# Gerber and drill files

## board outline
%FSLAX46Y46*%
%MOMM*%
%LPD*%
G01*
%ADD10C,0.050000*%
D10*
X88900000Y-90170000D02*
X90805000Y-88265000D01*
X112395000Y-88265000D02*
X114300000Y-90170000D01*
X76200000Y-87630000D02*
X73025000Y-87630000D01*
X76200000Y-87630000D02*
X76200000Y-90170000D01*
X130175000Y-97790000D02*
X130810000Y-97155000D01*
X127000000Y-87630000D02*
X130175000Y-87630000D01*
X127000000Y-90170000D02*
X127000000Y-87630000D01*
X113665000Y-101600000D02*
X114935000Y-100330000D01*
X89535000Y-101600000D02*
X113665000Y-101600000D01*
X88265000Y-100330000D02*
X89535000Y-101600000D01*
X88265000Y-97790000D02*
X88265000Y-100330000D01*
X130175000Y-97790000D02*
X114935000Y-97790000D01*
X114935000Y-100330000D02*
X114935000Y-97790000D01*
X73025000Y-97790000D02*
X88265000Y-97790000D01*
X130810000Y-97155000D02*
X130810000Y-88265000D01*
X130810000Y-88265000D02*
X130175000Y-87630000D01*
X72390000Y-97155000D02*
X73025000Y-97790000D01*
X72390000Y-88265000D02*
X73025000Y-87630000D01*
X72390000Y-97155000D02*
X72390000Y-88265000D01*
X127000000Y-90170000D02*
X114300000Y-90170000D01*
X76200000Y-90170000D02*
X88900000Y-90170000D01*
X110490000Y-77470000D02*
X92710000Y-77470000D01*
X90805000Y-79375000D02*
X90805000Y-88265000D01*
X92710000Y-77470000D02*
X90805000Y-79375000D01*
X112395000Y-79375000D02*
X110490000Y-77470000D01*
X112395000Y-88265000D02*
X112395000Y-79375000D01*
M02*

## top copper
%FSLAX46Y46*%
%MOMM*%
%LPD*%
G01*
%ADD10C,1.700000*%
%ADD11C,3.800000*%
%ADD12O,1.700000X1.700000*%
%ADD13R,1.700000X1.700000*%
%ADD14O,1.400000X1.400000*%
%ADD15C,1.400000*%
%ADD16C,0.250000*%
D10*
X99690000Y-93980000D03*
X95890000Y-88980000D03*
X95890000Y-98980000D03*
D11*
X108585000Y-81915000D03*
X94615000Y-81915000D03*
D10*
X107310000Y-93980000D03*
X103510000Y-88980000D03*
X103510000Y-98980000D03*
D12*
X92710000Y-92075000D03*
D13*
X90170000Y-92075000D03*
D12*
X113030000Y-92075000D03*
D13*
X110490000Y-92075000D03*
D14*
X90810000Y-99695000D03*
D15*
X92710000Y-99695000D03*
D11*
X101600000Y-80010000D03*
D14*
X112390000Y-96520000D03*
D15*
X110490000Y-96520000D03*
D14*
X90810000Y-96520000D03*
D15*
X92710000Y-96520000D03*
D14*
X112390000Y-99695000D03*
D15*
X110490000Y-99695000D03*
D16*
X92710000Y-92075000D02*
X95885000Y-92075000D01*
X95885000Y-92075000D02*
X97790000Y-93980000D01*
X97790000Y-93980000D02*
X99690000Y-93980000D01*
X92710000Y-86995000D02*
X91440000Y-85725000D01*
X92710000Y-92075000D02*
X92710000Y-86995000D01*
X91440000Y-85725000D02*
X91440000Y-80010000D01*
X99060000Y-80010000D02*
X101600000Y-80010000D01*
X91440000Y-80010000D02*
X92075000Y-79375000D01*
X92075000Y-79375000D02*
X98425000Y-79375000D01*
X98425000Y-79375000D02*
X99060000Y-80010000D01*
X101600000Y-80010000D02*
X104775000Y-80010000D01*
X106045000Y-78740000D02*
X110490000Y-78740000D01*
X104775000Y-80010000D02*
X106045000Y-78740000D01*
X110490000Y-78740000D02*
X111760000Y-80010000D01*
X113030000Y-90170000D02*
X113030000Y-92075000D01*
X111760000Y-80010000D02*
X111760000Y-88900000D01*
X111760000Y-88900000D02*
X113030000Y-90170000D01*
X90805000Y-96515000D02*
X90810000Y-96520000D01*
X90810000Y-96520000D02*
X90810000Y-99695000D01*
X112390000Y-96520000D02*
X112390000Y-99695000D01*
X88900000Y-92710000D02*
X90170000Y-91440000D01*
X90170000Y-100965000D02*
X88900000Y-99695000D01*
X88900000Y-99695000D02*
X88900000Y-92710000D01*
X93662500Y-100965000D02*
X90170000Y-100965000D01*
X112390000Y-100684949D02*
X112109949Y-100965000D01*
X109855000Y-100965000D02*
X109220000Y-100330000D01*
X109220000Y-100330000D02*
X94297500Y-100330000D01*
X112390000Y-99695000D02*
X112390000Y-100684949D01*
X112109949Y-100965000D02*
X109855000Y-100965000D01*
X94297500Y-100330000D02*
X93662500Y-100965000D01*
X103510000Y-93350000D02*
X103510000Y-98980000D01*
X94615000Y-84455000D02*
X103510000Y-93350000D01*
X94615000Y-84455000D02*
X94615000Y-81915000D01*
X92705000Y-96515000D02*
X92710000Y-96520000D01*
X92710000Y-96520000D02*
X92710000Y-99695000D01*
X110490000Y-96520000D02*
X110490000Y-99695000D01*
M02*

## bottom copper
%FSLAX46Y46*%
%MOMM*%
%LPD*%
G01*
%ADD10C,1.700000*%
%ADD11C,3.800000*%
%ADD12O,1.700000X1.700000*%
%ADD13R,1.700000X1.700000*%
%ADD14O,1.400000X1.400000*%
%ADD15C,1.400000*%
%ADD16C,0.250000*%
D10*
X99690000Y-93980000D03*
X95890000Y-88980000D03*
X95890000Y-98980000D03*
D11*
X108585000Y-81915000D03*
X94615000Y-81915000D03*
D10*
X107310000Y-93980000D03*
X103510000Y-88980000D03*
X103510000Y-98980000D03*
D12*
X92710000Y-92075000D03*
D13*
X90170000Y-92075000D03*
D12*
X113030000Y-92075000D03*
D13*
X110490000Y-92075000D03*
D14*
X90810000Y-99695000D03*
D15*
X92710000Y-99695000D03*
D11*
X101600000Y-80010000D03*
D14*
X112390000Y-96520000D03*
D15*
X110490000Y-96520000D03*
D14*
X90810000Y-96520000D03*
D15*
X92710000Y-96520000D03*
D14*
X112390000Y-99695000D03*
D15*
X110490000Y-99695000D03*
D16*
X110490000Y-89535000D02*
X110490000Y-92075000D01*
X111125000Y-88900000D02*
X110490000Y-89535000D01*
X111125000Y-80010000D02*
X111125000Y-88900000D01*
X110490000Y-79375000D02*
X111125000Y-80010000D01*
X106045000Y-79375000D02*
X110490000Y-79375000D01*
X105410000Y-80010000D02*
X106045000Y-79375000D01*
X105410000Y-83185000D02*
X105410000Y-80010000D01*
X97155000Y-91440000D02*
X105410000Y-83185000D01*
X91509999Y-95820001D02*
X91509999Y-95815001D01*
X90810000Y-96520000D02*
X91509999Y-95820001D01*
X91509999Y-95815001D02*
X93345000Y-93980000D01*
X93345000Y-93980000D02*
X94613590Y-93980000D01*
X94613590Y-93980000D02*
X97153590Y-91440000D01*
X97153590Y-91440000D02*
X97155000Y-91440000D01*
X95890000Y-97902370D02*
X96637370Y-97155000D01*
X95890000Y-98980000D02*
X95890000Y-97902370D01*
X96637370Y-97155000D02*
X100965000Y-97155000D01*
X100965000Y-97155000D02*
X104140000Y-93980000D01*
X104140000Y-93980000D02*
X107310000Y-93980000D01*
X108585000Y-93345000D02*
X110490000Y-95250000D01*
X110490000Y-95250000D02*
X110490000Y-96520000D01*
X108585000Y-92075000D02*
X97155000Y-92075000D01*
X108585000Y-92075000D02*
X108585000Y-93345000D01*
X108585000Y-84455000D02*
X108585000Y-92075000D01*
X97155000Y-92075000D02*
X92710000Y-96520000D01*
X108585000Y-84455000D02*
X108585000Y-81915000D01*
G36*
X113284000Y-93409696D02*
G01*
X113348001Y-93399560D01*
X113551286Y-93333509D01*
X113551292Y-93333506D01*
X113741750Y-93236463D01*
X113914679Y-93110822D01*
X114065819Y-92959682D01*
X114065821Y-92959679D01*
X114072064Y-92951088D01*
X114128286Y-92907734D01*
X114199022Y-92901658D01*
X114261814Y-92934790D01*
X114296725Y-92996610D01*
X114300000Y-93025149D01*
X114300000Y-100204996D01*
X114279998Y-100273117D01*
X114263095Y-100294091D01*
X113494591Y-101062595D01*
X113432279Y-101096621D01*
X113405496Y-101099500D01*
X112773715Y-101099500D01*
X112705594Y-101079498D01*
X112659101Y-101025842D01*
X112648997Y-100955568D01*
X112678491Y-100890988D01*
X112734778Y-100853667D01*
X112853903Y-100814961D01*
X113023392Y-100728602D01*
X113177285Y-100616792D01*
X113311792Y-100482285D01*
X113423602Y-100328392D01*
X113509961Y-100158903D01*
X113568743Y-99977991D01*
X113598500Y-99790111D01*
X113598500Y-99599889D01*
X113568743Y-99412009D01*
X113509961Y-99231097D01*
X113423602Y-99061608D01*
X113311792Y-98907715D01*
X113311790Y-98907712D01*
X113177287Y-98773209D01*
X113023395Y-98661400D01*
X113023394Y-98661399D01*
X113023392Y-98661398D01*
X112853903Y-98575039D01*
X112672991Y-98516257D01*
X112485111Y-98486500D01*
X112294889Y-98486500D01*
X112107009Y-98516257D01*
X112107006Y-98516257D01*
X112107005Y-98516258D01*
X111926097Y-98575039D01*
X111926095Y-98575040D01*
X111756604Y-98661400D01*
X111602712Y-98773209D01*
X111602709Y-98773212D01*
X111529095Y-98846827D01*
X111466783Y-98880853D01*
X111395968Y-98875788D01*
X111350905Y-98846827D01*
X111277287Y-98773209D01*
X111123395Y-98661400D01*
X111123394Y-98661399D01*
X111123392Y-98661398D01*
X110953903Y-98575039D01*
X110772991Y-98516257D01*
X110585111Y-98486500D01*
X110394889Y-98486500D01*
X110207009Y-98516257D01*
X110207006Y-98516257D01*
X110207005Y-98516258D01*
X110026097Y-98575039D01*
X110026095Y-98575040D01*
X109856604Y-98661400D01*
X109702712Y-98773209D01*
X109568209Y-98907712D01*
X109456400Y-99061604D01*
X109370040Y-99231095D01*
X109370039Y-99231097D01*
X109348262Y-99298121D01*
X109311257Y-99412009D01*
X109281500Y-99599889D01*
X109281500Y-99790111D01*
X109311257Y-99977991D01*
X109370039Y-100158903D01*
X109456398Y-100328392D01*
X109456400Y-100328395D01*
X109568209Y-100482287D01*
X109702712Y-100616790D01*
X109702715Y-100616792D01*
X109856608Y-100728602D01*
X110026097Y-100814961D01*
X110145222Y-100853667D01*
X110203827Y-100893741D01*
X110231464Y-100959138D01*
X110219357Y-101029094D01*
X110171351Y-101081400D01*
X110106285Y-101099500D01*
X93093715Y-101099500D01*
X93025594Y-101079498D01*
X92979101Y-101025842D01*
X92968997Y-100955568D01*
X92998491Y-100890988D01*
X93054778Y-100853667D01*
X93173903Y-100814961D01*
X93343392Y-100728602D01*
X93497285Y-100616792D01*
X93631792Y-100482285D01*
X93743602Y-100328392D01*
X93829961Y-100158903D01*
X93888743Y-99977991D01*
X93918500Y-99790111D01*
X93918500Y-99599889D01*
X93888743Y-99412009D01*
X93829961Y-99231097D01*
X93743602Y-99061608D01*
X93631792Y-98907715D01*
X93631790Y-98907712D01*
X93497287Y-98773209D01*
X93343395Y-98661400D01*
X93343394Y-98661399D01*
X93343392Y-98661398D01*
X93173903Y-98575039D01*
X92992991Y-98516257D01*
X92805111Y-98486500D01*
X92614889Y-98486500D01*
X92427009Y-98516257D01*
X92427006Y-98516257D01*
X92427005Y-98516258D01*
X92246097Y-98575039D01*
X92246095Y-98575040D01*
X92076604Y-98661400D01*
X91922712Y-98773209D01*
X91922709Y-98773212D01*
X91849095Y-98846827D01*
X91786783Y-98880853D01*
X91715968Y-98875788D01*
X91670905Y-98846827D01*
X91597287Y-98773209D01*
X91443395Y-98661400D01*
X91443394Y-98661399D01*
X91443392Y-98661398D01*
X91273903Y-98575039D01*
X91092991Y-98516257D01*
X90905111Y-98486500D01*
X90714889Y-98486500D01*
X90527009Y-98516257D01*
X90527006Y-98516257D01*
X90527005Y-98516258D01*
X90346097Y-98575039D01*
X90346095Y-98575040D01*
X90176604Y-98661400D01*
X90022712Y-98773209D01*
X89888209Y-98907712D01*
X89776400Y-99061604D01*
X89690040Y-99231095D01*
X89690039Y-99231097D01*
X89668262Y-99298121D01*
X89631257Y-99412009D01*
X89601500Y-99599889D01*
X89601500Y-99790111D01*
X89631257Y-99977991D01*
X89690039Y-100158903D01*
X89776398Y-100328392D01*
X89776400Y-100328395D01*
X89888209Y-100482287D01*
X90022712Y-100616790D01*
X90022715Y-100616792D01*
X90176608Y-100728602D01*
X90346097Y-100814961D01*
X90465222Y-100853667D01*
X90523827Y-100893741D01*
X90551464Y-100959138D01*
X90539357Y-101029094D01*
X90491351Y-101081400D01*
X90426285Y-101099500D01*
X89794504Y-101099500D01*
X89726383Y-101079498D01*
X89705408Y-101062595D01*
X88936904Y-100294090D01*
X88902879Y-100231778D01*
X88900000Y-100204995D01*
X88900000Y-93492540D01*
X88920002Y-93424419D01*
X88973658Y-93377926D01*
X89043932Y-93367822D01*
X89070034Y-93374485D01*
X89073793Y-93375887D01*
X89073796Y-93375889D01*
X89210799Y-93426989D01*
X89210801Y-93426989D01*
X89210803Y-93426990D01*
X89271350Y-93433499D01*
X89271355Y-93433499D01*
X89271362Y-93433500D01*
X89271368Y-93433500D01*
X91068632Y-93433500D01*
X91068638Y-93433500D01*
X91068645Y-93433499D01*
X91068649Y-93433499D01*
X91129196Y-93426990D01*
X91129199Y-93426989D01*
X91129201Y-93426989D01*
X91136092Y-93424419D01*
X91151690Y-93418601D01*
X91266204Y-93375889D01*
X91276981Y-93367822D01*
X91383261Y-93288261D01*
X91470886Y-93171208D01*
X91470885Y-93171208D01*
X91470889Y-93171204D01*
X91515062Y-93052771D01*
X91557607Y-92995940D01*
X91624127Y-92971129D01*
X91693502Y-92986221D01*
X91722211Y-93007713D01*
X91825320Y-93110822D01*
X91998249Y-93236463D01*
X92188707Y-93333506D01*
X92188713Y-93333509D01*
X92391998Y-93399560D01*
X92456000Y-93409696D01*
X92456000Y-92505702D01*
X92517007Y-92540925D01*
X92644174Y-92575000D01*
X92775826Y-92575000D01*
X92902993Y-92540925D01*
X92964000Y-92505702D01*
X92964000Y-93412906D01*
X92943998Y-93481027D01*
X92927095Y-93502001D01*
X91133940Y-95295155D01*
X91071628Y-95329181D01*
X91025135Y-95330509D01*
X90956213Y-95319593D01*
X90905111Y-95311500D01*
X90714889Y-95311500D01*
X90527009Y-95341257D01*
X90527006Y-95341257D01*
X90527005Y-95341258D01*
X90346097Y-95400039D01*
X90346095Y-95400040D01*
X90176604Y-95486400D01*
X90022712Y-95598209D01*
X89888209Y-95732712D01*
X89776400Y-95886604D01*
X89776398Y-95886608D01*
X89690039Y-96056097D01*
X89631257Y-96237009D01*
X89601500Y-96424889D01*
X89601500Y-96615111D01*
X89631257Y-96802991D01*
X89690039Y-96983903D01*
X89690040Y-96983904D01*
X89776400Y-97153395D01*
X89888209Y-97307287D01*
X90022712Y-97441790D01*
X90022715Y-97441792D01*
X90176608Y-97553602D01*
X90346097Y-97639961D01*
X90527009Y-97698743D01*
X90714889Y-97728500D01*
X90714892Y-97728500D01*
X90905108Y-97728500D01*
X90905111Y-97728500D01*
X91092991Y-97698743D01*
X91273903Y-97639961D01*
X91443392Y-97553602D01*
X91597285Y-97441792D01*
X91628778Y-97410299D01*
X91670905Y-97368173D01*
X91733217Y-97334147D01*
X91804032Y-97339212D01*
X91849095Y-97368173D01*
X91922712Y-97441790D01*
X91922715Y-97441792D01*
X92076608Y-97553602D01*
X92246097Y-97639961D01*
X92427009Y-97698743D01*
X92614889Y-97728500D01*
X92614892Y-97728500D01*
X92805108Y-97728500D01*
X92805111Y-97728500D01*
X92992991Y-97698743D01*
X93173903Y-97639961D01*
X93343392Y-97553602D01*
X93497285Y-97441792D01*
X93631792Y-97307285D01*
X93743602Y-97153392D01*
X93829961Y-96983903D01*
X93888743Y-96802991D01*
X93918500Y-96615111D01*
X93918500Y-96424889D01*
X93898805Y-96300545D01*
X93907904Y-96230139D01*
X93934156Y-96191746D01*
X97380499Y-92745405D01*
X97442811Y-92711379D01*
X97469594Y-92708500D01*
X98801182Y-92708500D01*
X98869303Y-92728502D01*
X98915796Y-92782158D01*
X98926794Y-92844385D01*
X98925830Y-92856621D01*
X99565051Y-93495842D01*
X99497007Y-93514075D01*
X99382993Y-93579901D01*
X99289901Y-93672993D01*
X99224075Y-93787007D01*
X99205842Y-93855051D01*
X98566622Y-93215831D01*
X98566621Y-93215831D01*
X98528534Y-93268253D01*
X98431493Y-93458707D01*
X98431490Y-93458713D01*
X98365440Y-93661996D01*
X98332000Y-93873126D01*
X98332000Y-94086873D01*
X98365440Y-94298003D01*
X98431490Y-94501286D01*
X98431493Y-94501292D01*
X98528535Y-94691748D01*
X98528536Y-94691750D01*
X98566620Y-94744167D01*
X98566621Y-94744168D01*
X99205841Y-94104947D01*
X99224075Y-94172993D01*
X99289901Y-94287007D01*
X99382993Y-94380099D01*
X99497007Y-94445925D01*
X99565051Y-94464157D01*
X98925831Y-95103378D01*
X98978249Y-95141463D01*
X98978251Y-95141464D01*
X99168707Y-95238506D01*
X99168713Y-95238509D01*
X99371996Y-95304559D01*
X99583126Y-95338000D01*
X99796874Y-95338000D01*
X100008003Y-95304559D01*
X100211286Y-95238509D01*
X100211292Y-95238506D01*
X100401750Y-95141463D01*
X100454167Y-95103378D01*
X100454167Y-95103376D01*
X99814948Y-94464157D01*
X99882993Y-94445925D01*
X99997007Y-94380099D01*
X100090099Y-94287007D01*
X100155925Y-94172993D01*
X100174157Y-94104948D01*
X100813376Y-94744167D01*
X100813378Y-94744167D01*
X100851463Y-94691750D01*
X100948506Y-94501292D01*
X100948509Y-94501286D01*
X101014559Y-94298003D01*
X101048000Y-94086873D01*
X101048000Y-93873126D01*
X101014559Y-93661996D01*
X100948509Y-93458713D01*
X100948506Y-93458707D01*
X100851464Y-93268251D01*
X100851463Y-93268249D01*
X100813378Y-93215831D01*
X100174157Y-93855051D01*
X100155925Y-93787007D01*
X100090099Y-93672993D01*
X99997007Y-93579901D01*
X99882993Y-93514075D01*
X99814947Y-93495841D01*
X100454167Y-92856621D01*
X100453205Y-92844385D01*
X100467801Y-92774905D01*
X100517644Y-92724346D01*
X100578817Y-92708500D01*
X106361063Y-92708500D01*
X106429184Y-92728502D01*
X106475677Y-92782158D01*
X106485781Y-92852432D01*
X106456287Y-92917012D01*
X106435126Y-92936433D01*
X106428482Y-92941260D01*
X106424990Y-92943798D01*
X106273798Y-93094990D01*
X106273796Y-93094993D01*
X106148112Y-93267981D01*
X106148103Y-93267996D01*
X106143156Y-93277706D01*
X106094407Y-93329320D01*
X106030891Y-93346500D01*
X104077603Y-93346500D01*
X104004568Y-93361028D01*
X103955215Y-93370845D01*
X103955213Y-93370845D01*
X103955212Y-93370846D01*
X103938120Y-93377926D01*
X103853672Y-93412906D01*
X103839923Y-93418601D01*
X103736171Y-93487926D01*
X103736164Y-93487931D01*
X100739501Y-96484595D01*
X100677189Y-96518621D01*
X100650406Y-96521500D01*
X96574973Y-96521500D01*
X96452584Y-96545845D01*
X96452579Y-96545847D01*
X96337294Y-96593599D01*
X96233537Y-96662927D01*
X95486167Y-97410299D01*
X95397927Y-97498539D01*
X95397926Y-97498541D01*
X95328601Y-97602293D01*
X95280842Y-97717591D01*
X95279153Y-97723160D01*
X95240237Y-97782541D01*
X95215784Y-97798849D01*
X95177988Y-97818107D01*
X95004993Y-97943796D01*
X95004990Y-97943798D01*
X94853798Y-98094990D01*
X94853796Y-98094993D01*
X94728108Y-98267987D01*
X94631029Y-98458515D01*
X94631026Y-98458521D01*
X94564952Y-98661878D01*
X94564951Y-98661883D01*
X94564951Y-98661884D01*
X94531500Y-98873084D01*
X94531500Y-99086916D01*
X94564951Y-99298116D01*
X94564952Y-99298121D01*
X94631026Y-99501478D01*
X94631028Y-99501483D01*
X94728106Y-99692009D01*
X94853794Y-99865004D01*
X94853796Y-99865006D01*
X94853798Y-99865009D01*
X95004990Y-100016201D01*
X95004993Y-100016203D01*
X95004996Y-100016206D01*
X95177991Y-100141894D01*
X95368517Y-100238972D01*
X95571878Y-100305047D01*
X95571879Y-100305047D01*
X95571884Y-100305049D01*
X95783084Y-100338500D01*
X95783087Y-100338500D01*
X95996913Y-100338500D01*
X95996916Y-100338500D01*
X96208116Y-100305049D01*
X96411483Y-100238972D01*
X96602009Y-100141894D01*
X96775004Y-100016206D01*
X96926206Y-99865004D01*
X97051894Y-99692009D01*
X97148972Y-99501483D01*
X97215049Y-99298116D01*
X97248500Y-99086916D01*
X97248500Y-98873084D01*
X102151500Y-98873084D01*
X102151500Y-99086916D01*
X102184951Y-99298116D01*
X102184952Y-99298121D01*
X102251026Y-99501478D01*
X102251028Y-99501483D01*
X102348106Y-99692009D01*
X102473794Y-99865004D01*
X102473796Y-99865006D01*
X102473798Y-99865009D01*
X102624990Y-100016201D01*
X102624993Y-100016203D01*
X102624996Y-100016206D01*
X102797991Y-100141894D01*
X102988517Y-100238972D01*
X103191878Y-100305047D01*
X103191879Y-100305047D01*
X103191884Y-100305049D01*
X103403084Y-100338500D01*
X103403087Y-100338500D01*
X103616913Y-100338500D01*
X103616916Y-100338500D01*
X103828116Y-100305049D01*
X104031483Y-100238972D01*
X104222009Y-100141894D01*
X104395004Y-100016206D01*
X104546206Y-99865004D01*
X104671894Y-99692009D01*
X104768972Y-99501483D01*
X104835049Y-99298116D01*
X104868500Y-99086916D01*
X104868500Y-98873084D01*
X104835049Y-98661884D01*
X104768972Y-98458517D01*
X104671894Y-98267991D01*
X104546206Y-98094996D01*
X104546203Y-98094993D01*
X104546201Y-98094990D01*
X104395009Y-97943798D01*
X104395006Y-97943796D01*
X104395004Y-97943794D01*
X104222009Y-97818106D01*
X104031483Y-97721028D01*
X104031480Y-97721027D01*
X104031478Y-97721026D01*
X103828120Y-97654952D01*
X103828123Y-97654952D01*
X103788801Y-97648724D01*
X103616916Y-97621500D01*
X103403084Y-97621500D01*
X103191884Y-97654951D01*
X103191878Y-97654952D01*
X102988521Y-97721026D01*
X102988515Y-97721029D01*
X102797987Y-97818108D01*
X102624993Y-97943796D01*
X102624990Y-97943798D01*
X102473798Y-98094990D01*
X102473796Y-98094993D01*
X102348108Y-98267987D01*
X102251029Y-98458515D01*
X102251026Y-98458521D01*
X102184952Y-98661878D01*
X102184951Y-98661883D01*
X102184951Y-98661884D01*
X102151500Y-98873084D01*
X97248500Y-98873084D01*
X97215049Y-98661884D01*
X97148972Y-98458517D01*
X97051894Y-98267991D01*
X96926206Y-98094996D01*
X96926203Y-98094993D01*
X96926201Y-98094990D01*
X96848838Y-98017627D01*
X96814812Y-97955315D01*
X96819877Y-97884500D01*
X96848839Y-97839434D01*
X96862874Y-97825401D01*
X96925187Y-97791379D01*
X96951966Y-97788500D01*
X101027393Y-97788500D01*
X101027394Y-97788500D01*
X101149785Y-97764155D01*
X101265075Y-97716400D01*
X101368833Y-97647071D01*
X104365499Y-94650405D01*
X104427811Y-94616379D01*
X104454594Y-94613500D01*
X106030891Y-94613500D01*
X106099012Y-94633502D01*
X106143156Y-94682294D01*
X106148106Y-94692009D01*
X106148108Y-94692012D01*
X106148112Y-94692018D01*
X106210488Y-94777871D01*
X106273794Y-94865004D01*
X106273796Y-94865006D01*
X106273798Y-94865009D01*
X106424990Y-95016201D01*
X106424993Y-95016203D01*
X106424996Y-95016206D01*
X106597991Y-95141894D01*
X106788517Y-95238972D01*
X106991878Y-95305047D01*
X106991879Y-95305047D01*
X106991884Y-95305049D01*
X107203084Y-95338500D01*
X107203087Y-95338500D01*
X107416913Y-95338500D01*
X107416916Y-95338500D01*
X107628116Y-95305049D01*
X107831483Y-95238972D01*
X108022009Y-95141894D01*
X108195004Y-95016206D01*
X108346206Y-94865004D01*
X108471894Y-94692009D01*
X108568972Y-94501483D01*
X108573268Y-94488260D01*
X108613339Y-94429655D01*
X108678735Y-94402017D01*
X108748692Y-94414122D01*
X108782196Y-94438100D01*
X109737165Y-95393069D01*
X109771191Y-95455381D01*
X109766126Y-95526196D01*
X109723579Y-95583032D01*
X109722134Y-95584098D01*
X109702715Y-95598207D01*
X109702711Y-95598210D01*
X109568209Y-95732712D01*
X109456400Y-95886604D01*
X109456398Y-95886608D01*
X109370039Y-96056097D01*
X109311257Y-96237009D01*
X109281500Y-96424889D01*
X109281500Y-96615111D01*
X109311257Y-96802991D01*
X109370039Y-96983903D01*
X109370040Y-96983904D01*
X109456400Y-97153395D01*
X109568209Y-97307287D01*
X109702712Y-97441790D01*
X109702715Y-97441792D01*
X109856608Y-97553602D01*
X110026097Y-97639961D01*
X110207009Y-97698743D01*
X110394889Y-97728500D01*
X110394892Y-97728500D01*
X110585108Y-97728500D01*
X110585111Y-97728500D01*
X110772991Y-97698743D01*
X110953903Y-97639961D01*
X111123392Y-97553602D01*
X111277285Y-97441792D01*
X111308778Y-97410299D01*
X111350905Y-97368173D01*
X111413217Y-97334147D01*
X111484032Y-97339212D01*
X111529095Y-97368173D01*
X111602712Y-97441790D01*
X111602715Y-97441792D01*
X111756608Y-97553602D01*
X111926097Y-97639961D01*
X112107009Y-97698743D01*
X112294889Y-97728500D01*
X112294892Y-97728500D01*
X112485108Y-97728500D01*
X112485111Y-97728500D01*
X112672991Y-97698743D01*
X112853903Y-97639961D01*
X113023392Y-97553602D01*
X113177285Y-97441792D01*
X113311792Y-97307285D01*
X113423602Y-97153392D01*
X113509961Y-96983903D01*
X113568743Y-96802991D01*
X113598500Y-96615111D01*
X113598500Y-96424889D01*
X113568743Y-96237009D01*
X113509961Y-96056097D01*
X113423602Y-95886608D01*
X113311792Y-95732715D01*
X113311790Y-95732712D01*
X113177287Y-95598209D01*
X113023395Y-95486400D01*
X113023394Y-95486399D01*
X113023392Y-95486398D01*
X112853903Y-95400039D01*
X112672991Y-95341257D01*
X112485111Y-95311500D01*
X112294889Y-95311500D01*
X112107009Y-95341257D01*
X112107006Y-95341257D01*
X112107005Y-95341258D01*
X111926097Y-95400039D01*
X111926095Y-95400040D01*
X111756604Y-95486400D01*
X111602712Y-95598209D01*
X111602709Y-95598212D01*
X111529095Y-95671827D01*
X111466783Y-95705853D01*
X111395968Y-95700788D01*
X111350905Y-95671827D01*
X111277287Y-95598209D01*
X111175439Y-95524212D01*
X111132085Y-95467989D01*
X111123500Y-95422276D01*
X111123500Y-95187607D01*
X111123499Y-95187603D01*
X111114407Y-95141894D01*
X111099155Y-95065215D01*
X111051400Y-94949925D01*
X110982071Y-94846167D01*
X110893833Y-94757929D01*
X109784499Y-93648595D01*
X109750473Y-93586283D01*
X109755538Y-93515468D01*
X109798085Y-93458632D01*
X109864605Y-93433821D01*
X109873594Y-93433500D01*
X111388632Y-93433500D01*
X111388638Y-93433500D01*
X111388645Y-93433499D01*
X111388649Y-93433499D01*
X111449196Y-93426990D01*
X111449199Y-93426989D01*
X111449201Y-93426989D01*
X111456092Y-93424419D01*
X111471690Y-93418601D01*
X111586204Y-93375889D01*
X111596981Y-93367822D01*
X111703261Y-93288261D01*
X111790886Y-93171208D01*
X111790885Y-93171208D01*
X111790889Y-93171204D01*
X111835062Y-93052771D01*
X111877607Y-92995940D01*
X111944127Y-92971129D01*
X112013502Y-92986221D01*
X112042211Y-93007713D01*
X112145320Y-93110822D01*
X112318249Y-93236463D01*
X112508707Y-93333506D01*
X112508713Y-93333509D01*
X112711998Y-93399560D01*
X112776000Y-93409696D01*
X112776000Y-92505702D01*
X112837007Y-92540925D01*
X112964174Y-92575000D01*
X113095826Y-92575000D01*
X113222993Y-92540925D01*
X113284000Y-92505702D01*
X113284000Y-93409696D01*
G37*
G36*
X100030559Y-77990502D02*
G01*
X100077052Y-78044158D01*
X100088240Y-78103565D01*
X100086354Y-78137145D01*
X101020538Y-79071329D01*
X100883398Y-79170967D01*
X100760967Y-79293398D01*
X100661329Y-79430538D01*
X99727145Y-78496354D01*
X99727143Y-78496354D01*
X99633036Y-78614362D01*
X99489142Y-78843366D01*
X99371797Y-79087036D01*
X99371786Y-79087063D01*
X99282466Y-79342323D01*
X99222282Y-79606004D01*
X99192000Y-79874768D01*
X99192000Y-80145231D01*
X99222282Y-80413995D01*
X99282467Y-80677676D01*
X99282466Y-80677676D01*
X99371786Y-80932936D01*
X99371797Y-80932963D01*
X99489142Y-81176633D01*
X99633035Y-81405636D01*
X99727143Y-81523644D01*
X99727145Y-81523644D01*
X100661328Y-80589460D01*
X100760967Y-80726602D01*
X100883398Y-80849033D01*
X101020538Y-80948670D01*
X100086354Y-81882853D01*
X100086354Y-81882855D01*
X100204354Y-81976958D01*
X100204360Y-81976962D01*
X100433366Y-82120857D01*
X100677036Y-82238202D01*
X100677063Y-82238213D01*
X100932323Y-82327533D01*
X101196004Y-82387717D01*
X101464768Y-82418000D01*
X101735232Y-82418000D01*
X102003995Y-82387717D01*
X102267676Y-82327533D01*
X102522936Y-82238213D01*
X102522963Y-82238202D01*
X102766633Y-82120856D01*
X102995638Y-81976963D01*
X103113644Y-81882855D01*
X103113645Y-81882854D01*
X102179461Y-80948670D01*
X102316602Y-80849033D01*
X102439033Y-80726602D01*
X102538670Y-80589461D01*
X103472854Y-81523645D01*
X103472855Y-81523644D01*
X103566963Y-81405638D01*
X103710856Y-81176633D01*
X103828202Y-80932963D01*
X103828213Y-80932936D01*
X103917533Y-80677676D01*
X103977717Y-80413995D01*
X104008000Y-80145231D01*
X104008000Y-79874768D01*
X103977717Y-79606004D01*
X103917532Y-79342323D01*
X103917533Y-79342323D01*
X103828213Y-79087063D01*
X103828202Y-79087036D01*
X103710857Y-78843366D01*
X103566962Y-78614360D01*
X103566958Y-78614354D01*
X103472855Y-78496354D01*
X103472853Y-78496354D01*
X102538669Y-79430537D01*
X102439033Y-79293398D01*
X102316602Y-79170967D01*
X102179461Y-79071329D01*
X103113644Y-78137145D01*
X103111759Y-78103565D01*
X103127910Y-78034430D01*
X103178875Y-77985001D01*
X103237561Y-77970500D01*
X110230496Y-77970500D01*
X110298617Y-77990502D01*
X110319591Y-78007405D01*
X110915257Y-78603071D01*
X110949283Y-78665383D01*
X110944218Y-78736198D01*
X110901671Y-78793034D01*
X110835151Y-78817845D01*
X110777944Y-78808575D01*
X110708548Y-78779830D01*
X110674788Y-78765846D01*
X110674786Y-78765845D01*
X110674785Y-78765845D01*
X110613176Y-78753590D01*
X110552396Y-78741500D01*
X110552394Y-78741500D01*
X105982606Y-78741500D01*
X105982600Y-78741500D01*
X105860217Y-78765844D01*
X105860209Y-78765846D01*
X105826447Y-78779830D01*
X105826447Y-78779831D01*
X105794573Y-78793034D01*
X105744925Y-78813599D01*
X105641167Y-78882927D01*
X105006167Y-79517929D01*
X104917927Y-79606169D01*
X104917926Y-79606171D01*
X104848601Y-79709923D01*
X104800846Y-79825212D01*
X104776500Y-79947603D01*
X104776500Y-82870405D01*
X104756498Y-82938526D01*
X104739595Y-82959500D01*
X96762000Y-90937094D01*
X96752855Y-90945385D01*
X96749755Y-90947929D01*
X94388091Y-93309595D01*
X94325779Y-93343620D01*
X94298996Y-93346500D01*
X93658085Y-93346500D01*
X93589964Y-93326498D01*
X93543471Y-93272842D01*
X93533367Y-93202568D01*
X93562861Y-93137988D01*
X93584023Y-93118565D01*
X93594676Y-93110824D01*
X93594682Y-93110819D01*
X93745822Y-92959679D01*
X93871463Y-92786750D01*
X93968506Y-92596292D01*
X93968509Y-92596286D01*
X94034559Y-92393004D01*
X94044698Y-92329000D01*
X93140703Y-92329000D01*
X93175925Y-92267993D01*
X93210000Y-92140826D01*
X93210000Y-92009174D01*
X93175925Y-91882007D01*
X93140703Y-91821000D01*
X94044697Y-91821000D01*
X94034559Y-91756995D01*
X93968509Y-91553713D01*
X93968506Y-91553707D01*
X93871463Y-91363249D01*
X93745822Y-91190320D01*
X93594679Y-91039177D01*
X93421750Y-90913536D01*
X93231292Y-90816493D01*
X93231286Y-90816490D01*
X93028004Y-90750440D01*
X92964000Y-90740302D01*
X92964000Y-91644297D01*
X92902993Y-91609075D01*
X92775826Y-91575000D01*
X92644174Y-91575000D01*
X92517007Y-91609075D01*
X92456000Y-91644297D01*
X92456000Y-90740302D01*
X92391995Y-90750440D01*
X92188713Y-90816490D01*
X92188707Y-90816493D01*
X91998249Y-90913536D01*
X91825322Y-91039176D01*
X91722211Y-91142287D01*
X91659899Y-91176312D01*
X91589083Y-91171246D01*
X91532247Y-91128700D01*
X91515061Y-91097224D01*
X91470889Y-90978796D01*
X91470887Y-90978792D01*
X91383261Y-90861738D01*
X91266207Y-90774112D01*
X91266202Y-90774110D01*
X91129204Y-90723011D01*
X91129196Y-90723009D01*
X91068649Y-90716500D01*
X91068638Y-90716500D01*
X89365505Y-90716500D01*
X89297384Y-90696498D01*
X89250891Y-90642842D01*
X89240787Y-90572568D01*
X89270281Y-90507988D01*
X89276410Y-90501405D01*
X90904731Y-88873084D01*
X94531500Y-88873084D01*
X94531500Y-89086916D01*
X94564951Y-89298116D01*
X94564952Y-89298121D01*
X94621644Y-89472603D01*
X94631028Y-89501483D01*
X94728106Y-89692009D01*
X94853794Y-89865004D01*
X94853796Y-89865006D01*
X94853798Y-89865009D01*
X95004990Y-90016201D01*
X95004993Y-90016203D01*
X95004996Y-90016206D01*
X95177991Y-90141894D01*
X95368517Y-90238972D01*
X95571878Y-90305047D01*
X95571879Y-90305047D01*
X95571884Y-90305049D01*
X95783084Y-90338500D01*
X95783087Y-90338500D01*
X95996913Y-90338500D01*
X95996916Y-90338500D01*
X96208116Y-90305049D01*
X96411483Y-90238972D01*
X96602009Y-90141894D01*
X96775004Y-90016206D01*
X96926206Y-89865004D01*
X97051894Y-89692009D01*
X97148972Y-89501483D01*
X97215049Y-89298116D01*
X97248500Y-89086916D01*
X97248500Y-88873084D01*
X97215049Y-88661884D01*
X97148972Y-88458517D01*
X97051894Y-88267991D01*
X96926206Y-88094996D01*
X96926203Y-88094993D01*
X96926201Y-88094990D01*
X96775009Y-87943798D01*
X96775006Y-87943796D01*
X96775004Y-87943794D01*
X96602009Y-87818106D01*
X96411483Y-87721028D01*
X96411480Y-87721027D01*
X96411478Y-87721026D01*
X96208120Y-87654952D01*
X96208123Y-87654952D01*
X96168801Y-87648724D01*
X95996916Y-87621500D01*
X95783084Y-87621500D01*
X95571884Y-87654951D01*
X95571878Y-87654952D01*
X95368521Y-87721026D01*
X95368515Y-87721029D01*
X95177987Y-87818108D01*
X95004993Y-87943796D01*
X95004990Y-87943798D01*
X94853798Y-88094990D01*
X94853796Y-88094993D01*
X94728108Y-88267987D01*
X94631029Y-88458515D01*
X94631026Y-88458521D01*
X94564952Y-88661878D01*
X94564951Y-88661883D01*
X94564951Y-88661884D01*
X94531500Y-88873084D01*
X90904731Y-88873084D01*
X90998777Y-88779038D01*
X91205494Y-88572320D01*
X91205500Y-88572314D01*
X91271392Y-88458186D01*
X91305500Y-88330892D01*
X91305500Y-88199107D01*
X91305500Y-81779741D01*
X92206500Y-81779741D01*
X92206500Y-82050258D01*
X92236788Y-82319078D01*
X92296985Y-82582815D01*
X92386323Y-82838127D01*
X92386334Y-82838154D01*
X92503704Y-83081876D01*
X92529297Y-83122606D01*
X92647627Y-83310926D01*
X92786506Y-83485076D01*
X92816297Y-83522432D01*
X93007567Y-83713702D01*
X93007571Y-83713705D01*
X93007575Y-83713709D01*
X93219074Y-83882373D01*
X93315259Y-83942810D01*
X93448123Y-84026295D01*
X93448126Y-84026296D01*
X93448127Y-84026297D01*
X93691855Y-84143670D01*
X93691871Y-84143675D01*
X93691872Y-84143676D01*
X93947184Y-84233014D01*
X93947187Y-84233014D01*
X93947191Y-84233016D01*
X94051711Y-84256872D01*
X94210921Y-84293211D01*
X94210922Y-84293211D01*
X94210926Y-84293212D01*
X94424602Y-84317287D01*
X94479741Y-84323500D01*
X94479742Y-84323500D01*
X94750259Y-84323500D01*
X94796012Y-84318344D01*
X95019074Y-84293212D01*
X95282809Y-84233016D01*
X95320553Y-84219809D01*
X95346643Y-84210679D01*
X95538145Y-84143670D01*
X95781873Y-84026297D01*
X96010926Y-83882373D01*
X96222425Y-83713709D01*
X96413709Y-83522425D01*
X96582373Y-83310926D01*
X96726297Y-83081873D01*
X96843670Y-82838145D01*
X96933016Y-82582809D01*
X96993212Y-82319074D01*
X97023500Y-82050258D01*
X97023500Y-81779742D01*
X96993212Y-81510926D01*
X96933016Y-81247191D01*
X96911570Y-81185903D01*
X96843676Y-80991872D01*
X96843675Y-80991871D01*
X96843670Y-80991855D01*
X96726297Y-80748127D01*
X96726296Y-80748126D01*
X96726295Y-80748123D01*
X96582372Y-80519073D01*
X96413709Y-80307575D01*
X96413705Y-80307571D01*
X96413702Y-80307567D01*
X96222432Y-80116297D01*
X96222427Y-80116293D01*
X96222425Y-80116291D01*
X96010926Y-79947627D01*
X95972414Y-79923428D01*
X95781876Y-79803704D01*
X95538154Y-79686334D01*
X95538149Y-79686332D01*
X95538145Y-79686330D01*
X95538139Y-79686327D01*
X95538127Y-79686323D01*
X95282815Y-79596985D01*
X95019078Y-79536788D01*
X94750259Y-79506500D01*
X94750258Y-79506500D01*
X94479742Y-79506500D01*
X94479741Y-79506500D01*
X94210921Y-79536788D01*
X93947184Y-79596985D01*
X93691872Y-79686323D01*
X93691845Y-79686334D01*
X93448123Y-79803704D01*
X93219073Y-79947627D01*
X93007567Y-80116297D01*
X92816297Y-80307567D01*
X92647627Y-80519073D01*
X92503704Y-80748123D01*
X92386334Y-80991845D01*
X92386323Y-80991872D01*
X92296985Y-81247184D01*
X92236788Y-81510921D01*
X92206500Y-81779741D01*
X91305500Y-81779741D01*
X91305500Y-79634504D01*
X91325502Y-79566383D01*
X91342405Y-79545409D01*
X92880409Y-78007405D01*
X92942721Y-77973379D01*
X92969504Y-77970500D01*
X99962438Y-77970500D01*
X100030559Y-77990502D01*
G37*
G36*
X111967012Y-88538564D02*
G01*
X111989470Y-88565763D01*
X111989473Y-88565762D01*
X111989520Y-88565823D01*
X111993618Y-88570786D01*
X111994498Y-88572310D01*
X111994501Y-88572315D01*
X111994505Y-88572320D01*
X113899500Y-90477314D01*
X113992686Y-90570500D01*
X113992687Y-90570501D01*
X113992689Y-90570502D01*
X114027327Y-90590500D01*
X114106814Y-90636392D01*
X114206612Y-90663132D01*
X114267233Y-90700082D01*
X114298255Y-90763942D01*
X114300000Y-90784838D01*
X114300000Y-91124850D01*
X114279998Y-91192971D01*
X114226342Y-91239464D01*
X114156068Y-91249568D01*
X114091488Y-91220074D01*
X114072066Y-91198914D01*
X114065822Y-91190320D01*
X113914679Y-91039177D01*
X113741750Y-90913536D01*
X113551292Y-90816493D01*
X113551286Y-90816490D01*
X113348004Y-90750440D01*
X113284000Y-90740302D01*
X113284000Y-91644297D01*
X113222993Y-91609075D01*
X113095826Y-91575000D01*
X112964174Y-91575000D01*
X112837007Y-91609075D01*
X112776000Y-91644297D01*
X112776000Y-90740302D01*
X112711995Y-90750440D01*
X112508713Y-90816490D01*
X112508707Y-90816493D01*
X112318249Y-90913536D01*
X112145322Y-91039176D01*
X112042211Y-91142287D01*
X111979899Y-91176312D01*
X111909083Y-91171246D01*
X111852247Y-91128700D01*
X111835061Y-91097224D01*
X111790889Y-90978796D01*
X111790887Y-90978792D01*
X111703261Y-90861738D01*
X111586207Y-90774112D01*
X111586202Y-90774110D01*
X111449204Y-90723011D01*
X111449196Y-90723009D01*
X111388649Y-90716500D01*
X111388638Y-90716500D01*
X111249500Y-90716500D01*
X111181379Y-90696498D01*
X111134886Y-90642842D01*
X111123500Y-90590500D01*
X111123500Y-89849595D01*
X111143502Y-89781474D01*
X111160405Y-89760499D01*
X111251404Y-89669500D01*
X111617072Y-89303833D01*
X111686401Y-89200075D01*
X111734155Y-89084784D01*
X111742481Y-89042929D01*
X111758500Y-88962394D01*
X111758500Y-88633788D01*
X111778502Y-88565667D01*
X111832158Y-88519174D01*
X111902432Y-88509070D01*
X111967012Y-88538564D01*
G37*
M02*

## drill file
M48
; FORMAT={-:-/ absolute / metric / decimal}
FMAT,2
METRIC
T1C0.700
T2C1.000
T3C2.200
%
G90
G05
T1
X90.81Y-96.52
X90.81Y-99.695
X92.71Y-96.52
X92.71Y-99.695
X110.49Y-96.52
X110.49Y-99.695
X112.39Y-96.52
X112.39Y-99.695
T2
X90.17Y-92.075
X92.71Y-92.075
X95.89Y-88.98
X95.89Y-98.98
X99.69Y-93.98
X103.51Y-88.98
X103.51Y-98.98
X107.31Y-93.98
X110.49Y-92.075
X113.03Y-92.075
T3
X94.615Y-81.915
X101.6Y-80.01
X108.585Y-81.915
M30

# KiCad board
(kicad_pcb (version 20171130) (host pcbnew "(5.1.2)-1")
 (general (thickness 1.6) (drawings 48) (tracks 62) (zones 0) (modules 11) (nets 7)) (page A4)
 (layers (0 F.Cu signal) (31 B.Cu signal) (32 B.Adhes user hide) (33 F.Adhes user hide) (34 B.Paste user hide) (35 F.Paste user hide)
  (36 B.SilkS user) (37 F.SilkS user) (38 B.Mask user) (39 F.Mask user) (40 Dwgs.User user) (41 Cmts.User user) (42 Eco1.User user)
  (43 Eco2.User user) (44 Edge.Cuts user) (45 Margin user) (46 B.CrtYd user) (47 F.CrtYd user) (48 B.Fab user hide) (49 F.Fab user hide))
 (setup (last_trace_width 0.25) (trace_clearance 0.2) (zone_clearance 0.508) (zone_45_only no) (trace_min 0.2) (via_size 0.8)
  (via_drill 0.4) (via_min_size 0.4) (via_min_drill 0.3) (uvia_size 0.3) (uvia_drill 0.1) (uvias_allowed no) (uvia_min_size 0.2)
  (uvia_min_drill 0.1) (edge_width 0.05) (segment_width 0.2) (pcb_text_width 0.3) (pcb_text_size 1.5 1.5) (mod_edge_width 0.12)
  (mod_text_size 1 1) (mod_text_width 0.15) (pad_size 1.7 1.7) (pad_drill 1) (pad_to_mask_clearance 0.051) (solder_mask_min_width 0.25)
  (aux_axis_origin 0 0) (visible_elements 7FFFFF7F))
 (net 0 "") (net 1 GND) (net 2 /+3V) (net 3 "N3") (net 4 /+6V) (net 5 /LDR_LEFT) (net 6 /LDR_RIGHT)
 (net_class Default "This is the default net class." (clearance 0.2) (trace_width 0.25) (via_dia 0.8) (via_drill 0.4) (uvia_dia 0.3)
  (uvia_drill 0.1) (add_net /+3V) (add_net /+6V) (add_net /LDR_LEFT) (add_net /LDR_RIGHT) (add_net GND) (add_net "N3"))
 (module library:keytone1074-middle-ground (layer F.Cu) (at 97.79 93.98 90)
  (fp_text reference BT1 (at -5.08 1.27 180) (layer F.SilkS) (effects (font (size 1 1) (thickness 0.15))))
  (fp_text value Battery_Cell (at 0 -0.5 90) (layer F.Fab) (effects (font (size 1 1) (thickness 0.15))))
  (pad 2 thru_hole circle (at 0 1.9 90) (size 1.7 1.7) (drill 1) (layers *.Cu *.Mask) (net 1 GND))
  (pad 3 thru_hole circle (at 5 -1.9 90) (size 1.7 1.7) (drill 1) (layers *.Cu *.Mask))
  (pad 1 thru_hole circle (at -5 -1.9 90) (size 1.7 1.7) (drill 1) (layers *.Cu *.Mask) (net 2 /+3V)))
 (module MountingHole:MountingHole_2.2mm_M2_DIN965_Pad (layer F.Cu) (at 108.585 81.915)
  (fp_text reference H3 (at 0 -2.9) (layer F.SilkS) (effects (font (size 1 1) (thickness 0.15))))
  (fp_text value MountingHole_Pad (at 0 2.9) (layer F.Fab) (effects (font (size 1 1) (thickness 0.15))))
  (pad 1 thru_hole circle (at 0 0) (size 3.8 3.8) (drill 2.2) (layers *.Cu *.Mask) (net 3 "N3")))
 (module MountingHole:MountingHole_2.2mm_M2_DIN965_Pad (layer F.Cu) (at 94.615 81.915)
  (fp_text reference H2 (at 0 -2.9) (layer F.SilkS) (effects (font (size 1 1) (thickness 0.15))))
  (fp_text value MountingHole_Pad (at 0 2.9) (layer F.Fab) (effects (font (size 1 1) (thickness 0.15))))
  (pad 1 thru_hole circle (at 0 0) (size 3.8 3.8) (drill 2.2) (layers *.Cu *.Mask) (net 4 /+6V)))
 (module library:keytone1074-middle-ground (layer F.Cu) (at 105.41 93.98 90)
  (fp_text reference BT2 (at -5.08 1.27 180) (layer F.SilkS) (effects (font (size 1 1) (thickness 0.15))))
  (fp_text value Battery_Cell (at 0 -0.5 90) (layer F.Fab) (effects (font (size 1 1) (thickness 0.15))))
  (pad 2 thru_hole circle (at 0 1.9 90) (size 1.7 1.7) (drill 1) (layers *.Cu *.Mask) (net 2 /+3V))
  (pad 3 thru_hole circle (at 5 -1.9 90) (size 1.7 1.7) (drill 1) (layers *.Cu *.Mask))
  (pad 1 thru_hole circle (at -5 -1.9 90) (size 1.7 1.7) (drill 1) (layers *.Cu *.Mask) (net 4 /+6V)))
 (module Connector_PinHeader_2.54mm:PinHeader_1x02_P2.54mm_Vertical (layer F.Cu) (at 90.17 92.075 90)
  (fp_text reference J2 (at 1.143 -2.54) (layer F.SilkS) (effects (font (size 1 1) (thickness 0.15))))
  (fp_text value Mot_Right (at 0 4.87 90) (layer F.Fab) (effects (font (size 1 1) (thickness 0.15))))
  (pad 2 thru_hole oval (at 0 2.54 90) (size 1.7 1.7) (drill 1) (layers *.Cu *.Mask) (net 1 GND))
  (pad 1 thru_hole rect (at 0 0 90) (size 1.7 1.7) (drill 1) (layers *.Cu *.Mask) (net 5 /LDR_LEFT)))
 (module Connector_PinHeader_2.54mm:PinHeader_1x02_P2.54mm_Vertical (layer F.Cu) (at 110.49 92.075 90)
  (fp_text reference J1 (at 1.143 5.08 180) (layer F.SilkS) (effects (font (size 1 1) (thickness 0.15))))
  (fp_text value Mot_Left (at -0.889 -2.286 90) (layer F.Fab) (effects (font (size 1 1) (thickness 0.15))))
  (pad 2 thru_hole oval (at 0 2.54 90) (size 1.7 1.7) (drill 1) (layers *.Cu *.Mask) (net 1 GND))
  (pad 1 thru_hole rect (at 0 0 90) (size 1.7 1.7) (drill 1) (layers *.Cu *.Mask) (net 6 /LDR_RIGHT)))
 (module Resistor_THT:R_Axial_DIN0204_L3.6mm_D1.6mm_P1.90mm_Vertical (layer F.Cu) (at 92.71 99.695 180)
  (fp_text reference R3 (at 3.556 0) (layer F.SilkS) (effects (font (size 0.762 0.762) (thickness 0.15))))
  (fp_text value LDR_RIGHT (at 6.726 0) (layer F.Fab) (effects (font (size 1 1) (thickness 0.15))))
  (pad 2 thru_hole oval (at 1.9 0 180) (size 1.4 1.4) (drill 0.7) (layers *.Cu *.Mask) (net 6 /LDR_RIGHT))
  (pad 1 thru_hole circle (at 0 0 180) (size 1.4 1.4) (drill 0.7) (layers *.Cu *.Mask) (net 3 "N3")))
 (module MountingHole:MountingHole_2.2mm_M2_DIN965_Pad (layer F.Cu) (at 101.6 80.01)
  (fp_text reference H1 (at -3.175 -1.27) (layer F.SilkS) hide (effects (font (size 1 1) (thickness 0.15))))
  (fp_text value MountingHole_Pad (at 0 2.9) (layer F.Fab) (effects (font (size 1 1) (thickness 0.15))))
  (pad 1 thru_hole circle (at 0 0) (size 3.8 3.8) (drill 2.2) (layers *.Cu *.Mask) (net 1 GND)))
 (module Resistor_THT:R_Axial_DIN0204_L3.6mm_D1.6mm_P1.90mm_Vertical (layer F.Cu) (at 110.49 96.52)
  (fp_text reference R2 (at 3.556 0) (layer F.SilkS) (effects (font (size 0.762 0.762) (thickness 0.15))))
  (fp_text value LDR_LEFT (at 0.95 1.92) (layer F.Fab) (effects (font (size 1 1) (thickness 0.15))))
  (pad 2 thru_hole oval (at 1.9 0) (size 1.4 1.4) (drill 0.7) (layers *.Cu *.Mask) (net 5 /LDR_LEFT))
  (pad 1 thru_hole circle (at 0 0) (size 1.4 1.4) (drill 0.7) (layers *.Cu *.Mask) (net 3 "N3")))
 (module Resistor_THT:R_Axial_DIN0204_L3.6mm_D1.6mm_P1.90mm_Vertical (layer F.Cu) (at 92.71 96.52 180)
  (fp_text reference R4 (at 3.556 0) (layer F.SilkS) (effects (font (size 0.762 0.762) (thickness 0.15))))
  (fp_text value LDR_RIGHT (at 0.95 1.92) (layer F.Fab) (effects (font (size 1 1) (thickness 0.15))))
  (pad 2 thru_hole oval (at 1.9 0 180) (size 1.4 1.4) (drill 0.7) (layers *.Cu *.Mask) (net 6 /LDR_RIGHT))
  (pad 1 thru_hole circle (at 0 0 180) (size 1.4 1.4) (drill 0.7) (layers *.Cu *.Mask) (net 3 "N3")))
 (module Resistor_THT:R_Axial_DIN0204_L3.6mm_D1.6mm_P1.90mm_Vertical (layer F.Cu) (at 110.49 99.695)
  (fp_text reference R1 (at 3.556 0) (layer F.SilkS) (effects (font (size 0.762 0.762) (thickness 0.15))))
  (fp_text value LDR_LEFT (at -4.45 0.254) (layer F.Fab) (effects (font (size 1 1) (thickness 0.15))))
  (pad 2 thru_hole oval (at 1.9 0) (size 1.4 1.4) (drill 0.7) (layers *.Cu *.Mask) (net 5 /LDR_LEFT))
  (pad 1 thru_hole circle (at 0 0) (size 1.4 1.4) (drill 0.7) (layers *.Cu *.Mask) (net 3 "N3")))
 (gr_line (start 88.9 90.17) (end 90.805 88.265) (layer Edge.Cuts) (width 0.05))
 (gr_line (start 112.395 88.265) (end 114.3 90.17) (layer Edge.Cuts) (width 0.05))
 (gr_line (start 76.2 87.63) (end 73.025 87.63) (layer Edge.Cuts) (width 0.05))
 (gr_line (start 76.2 87.63) (end 76.2 90.17) (layer Edge.Cuts) (width 0.05))
 (gr_line (start 130.175 97.79) (end 130.81 97.155) (layer Edge.Cuts) (width 0.05))
 (gr_line (start 127 87.63) (end 130.175 87.63) (layer Edge.Cuts) (width 0.05))
 (gr_line (start 127 90.17) (end 127 87.63) (layer Edge.Cuts) (width 0.05))
 (gr_line (start 113.665 101.6) (end 114.935 100.33) (layer Edge.Cuts) (width 0.05))
 (gr_line (start 89.535 101.6) (end 113.665 101.6) (layer Edge.Cuts) (width 0.05))
 (gr_line (start 88.265 100.33) (end 89.535 101.6) (layer Edge.Cuts) (width 0.05))
 (gr_line (start 88.265 97.79) (end 88.265 100.33) (layer Edge.Cuts) (width 0.05))
 (gr_line (start 130.175 97.79) (end 114.935 97.79) (layer Edge.Cuts) (width 0.05))
 (gr_line (start 114.935 100.33) (end 114.935 97.79) (layer Edge.Cuts) (width 0.05))
 (gr_line (start 73.025 97.79) (end 88.265 97.79) (layer Edge.Cuts) (width 0.05))
 (gr_line (start 130.81 97.155) (end 130.81 88.265) (layer Edge.Cuts) (width 0.05))
 (gr_line (start 130.81 88.265) (end 130.175 87.63) (layer Edge.Cuts) (width 0.05))
 (gr_line (start 72.39 97.155) (end 73.025 97.79) (layer Edge.Cuts) (width 0.05))
 (gr_line (start 72.39 88.265) (end 73.025 87.63) (layer Edge.Cuts) (width 0.05))
 (gr_line (start 72.39 97.155) (end 72.39 88.265) (layer Edge.Cuts) (width 0.05))
 (gr_line (start 127 90.17) (end 114.3 90.17) (layer Edge.Cuts) (width 0.05))
 (gr_line (start 76.2 90.17) (end 88.9 90.17) (layer Edge.Cuts) (width 0.05))
 (gr_line (start 110.49 77.47) (end 92.71 77.47) (layer Edge.Cuts) (width 0.05))
 (gr_line (start 90.805 79.375) (end 90.805 88.265) (layer Edge.Cuts) (width 0.05))
 (gr_line (start 92.71 77.47) (end 90.805 79.375) (layer Edge.Cuts) (width 0.05))
 (gr_line (start 112.395 79.375) (end 110.49 77.47) (layer Edge.Cuts) (width 0.05))
 (gr_line (start 112.395 88.265) (end 112.395 79.375) (layer Edge.Cuts) (width 0.05))
 (segment (start 92.71 92.075) (end 95.885 92.075) (width 0.25) (layer F.Cu) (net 1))
 (segment (start 95.885 92.075) (end 97.79 93.98) (width 0.25) (layer F.Cu) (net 1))
 (segment (start 97.79 93.98) (end 99.69 93.98) (width 0.25) (layer F.Cu) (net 1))
 (segment (start 92.71 86.995) (end 91.44 85.725) (width 0.25) (layer F.Cu) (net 1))
 (segment (start 92.71 92.075) (end 92.71 86.995) (width 0.25) (layer F.Cu) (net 1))
 (segment (start 91.44 85.725) (end 91.44 80.01) (width 0.25) (layer F.Cu) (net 1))
 (segment (start 99.06 80.01) (end 101.6 80.01) (width 0.25) (layer F.Cu) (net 1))
 (segment (start 91.44 80.01) (end 92.075 79.375) (width 0.25) (layer F.Cu) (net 1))
 (segment (start 92.075 79.375) (end 98.425 79.375) (width 0.25) (layer F.Cu) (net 1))
 (segment (start 98.425 79.375) (end 99.06 80.01) (width 0.25) (layer F.Cu) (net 1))
 (segment (start 101.6 80.01) (end 104.775 80.01) (width 0.25) (layer F.Cu) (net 1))
 (segment (start 106.045 78.74) (end 110.49 78.74) (width 0.25) (layer F.Cu) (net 1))
 (segment (start 104.775 80.01) (end 106.045 78.74) (width 0.25) (layer F.Cu) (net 1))
 (segment (start 110.49 78.74) (end 111.76 80.01) (width 0.25) (layer F.Cu) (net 1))
 (segment (start 113.03 90.17) (end 113.03 92.075) (width 0.25) (layer F.Cu) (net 1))
 (segment (start 111.76 80.01) (end 111.76 88.9) (width 0.25) (layer F.Cu) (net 1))
 (segment (start 111.76 88.9) (end 113.03 90.17) (width 0.25) (layer F.Cu) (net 1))
 (segment (start 90.805 96.515) (end 90.81 96.52) (width 0.25) (layer F.Cu) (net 6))
 (segment (start 90.81 96.52) (end 90.81 99.695) (width 0.25) (layer F.Cu) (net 6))
 (segment (start 110.49 89.535) (end 110.49 92.075) (width 0.25) (layer B.Cu) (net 6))
 (segment (start 111.125 88.9) (end 110.49 89.535) (width 0.25) (layer B.Cu) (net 6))
 (segment (start 111.125 80.01) (end 111.125 88.9) (width 0.25) (layer B.Cu) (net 6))
 (segment (start 110.49 79.375) (end 111.125 80.01) (width 0.25) (layer B.Cu) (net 6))
 (segment (start 106.045 79.375) (end 110.49 79.375) (width 0.25) (layer B.Cu) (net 6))
 (segment (start 105.41 80.01) (end 106.045 79.375) (width 0.25) (layer B.Cu) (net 6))
 (segment (start 105.41 83.185) (end 105.41 80.01) (width 0.25) (layer B.Cu) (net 6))
 (segment (start 97.155 91.44) (end 105.41 83.185) (width 0.25) (layer B.Cu) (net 6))
 (segment (start 91.509999 95.820001) (end 91.509999 95.815001) (width 0.25) (layer B.Cu) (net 6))
 (segment (start 90.81 96.52) (end 91.509999 95.820001) (width 0.25) (layer B.Cu) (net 6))
 (segment (start 91.509999 95.815001) (end 93.345 93.98) (width 0.25) (layer B.Cu) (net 6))
 (segment (start 93.345 93.98) (end 94.61359 93.98) (width 0.25) (layer B.Cu) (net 6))
 (segment (start 94.61359 93.98) (end 97.15359 91.44) (width 0.25) (layer B.Cu) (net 6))
 (segment (start 97.15359 91.44) (end 97.155 91.44) (width 0.25) (layer B.Cu) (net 6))
 (segment (start 112.39 96.52) (end 112.39 99.695) (width 0.25) (layer F.Cu) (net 5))
 (segment (start 88.9 92.71) (end 90.17 91.44) (width 0.25) (layer F.Cu) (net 5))
 (segment (start 90.17 100.965) (end 88.9 99.695) (width 0.25) (layer F.Cu) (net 5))
 (segment (start 88.9 99.695) (end 88.9 92.71) (width 0.25) (layer F.Cu) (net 5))
 (segment (start 93.6625 100.965) (end 90.17 100.965) (width 0.25) (layer F.Cu) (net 5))
 (segment (start 112.39 100.684949) (end 112.109949 100.965) (width 0.25) (layer F.Cu) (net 5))
 (segment (start 109.855 100.965) (end 109.22 100.33) (width 0.25) (layer F.Cu) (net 5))
 (segment (start 109.22 100.33) (end 94.2975 100.33) (width 0.25) (layer F.Cu) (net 5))
 (segment (start 112.39 99.695) (end 112.39 100.684949) (width 0.25) (layer F.Cu) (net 5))
 (segment (start 112.109949 100.965) (end 109.855 100.965) (width 0.25) (layer F.Cu) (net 5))
 (segment (start 94.2975 100.33) (end 93.6625 100.965) (width 0.25) (layer F.Cu) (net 5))
 (segment (start 95.89 97.90237) (end 96.63737 97.155) (width 0.25) (layer B.Cu) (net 2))
 (segment (start 95.89 98.98) (end 95.89 97.90237) (width 0.25) (layer B.Cu) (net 2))
 (segment (start 96.63737 97.155) (end 100.965 97.155) (width 0.25) (layer B.Cu) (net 2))
 (segment (start 100.965 97.155) (end 104.14 93.98) (width 0.25) (layer B.Cu) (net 2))
 (segment (start 104.14 93.98) (end 107.31 93.98) (width 0.25) (layer B.Cu) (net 2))
 (segment (start 103.51 93.35) (end 103.51 98.98) (width 0.25) (layer F.Cu) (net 4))
 (segment (start 94.615 84.455) (end 103.51 93.35) (width 0.25) (layer F.Cu) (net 4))
 (segment (start 94.615 84.455) (end 94.615 81.915) (width 0.25) (layer F.Cu) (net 4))
 (segment (start 92.705 96.515) (end 92.71 96.52) (width 0.25) (layer F.Cu) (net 3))
 (segment (start 92.71 96.52) (end 92.71 99.695) (width 0.25) (layer F.Cu) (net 3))
 (segment (start 110.49 96.52) (end 110.49 99.695) (width 0.25) (layer F.Cu) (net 3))
 (segment (start 108.585 93.345) (end 110.49 95.25) (width 0.25) (layer B.Cu) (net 3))
 (segment (start 110.49 95.25) (end 110.49 96.52) (width 0.25) (layer B.Cu) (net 3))
 (segment (start 108.585 92.075) (end 97.155 92.075) (width 0.25) (layer B.Cu) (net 3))
 (segment (start 108.585 92.075) (end 108.585 93.345) (width 0.25) (layer B.Cu) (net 3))
 (segment (start 108.585 84.455) (end 108.585 92.075) (width 0.25) (layer B.Cu) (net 3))
 (segment (start 97.155 92.075) (end 92.71 96.52) (width 0.25) (layer B.Cu) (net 3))
 (segment (start 108.585 84.455) (end 108.585 81.915) (width 0.25) (layer B.Cu) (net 3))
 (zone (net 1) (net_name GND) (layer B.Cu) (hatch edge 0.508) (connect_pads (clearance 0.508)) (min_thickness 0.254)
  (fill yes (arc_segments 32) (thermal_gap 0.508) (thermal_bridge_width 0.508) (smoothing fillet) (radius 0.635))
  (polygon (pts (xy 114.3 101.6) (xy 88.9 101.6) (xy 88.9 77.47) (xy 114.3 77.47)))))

